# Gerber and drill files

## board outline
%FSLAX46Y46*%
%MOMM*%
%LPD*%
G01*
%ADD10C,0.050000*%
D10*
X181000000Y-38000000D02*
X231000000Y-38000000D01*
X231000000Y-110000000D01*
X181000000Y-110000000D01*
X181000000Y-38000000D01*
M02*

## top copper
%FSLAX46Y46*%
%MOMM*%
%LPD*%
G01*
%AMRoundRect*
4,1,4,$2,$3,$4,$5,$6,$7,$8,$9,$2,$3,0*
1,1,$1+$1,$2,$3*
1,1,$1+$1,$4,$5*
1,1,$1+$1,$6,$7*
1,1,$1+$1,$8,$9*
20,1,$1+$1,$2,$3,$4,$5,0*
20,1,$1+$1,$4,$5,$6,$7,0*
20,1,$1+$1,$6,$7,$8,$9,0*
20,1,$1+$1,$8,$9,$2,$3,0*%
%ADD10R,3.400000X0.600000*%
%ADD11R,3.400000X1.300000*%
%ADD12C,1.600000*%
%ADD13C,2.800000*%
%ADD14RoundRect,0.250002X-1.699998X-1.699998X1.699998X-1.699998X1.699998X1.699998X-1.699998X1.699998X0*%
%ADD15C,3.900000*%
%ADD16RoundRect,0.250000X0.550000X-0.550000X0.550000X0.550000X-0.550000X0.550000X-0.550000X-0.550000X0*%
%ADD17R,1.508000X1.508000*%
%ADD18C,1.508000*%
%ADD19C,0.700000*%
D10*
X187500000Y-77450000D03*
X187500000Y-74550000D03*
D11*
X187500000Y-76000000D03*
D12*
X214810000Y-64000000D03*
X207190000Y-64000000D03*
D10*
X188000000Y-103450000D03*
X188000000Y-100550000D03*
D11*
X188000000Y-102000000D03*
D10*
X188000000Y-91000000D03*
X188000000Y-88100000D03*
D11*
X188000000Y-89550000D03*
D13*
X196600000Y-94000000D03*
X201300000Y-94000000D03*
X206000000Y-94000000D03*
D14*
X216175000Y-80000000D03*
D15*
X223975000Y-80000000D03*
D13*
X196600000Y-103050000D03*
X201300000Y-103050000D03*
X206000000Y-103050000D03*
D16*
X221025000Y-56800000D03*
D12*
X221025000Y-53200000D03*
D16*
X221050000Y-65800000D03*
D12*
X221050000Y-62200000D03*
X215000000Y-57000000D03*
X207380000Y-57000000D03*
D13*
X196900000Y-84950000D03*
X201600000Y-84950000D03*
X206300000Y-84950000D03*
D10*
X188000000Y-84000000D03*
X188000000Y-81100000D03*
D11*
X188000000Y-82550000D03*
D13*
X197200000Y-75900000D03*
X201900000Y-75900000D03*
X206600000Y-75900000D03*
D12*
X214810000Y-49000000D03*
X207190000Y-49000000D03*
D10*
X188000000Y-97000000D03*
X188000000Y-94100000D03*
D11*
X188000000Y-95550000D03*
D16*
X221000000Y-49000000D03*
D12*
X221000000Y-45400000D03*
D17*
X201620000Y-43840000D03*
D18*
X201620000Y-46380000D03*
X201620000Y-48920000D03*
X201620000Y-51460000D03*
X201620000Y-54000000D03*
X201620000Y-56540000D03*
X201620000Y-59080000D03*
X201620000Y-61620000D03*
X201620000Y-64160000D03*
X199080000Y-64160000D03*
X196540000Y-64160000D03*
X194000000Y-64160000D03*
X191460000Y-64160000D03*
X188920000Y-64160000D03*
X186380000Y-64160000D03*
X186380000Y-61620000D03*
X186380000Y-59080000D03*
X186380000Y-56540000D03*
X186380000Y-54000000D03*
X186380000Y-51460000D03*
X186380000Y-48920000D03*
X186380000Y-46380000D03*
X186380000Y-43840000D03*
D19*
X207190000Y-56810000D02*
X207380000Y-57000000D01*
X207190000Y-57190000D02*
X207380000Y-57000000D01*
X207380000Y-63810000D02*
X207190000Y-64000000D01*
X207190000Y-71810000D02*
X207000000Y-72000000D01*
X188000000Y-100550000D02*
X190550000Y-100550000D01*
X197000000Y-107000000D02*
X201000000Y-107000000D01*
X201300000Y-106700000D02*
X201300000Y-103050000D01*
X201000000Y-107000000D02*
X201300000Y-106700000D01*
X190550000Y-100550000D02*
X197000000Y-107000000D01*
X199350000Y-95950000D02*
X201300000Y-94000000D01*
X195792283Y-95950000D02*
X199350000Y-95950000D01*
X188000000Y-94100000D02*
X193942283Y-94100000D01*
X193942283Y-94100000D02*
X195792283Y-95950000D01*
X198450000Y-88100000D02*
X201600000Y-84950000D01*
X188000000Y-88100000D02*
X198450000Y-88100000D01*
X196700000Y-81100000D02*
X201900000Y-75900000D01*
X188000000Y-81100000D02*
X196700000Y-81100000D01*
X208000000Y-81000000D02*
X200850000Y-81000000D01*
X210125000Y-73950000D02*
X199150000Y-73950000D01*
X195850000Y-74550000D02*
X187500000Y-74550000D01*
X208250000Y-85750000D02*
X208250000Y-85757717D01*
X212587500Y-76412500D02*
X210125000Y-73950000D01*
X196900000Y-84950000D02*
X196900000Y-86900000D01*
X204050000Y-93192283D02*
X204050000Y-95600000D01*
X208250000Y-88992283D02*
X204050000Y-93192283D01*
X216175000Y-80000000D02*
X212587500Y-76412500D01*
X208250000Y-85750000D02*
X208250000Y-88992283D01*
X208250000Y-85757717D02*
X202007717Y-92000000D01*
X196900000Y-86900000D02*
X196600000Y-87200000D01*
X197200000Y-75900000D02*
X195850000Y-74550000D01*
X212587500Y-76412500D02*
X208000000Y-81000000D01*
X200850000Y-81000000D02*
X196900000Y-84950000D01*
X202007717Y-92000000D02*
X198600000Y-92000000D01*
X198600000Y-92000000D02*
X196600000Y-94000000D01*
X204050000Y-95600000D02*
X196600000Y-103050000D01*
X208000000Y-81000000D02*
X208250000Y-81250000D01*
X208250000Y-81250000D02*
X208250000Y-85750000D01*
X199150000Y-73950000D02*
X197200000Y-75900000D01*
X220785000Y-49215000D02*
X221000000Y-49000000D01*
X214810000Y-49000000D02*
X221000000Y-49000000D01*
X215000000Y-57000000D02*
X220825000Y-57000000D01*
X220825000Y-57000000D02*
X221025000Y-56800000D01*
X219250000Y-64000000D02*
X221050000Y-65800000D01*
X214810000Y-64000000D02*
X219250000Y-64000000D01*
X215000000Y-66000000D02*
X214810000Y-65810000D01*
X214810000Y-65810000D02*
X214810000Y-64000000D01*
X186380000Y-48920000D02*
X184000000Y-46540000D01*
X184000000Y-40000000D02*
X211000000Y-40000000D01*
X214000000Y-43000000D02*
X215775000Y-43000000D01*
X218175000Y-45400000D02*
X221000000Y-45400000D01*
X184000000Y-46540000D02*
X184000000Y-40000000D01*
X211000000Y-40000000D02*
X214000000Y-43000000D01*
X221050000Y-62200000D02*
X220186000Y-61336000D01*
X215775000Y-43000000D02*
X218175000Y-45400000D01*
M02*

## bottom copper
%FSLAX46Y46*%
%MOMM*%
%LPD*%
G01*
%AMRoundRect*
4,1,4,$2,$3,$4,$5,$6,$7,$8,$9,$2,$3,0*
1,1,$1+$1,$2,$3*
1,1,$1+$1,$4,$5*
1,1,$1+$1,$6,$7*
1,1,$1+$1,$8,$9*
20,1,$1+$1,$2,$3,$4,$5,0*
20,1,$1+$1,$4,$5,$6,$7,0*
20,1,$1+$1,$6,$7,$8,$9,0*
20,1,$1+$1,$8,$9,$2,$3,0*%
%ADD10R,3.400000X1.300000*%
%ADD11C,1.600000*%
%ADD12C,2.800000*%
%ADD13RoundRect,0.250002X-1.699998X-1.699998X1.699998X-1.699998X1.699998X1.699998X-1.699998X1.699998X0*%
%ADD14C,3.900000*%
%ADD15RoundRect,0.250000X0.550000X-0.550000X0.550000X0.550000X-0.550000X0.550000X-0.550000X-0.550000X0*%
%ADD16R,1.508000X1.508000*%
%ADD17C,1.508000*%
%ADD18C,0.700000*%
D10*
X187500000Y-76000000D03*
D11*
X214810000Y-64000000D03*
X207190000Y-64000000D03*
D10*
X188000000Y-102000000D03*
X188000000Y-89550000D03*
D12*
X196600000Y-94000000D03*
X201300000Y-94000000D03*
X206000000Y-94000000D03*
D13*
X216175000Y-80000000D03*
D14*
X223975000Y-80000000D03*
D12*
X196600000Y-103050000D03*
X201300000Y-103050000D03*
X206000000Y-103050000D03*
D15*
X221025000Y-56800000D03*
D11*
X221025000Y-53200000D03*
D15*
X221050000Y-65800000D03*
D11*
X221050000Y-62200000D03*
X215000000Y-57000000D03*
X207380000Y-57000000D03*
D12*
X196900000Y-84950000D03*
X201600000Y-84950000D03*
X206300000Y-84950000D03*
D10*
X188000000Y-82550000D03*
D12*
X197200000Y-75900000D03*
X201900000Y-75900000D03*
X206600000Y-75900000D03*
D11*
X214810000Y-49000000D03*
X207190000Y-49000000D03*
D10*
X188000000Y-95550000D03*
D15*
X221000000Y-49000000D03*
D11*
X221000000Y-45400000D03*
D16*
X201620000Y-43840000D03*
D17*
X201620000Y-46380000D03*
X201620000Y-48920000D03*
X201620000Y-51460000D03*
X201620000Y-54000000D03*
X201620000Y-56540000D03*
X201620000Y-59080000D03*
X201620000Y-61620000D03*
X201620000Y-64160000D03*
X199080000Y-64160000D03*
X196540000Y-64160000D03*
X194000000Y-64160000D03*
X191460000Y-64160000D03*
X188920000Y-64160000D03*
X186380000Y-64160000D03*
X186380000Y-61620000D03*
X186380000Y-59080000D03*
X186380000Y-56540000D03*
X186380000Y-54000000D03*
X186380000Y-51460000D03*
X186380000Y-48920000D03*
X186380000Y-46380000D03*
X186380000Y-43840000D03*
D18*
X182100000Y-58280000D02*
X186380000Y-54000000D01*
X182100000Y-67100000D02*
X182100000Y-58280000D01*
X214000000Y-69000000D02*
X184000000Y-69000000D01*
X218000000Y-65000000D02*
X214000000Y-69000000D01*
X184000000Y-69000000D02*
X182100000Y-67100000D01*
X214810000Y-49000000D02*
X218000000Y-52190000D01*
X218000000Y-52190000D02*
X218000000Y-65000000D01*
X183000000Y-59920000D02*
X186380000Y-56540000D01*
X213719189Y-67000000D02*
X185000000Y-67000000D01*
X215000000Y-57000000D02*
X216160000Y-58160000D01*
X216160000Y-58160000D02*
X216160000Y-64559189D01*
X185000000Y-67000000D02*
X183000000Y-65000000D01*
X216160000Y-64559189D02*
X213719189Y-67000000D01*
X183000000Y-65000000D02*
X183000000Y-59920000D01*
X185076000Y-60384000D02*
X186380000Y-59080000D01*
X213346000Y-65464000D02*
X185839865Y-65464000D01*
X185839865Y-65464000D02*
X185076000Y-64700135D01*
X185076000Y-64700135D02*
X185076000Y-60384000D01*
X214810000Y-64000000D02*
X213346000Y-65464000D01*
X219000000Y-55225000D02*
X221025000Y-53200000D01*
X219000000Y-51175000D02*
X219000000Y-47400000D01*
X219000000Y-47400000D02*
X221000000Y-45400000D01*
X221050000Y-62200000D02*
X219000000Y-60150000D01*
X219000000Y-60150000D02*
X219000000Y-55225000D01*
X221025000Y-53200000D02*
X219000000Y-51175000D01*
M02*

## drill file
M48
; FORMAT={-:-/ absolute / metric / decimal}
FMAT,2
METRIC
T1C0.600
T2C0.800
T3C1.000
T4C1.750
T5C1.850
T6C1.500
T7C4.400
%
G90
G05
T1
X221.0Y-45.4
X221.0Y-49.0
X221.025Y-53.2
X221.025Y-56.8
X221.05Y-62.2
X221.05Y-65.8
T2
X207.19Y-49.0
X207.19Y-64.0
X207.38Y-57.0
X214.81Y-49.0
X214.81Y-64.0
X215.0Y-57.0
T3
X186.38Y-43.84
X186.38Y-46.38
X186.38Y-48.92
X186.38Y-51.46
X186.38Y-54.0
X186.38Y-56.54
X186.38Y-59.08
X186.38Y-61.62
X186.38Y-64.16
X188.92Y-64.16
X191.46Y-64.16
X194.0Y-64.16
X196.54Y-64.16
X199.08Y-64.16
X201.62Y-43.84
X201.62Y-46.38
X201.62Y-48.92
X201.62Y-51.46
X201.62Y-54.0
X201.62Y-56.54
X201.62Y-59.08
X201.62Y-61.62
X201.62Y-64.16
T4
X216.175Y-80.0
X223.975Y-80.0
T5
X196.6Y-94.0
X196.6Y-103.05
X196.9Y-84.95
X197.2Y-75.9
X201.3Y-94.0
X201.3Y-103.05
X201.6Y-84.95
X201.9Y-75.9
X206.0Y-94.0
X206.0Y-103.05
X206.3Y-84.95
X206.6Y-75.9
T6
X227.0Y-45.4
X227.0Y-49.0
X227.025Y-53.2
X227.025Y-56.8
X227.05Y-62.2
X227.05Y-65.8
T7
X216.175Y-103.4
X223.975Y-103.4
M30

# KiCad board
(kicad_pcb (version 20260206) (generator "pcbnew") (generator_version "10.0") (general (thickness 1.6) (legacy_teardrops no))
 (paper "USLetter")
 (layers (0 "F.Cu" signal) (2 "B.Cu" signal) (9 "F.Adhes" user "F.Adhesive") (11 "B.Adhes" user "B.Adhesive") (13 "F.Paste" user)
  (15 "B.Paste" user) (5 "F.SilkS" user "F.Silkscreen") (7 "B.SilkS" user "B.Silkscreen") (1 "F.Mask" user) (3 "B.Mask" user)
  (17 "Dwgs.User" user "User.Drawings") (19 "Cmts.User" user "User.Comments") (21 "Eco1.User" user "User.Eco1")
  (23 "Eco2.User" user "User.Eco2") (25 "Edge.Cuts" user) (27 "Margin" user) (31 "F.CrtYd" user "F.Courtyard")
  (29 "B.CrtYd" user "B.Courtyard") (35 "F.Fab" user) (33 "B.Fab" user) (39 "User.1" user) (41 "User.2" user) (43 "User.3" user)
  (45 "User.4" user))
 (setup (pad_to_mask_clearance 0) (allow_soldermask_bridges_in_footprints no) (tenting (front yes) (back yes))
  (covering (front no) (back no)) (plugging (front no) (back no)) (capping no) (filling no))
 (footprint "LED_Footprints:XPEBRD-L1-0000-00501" (layer "F.Cu") (at 187.5 76 90)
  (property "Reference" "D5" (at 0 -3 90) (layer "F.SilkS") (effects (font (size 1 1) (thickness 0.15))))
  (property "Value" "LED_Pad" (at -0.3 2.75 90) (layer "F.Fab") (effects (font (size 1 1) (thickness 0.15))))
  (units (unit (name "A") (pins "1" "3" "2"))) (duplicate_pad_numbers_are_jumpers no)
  (pad "" smd rect (at 0 0 90) (size 1 3) (layers "F.Paste"))
  (pad "1" smd rect (at -1.45 0 90) (size 0.6 3.4) (layers "F.Cu" "F.Mask" "F.Paste") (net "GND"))
  (pad "2" smd rect (at 1.45 0 90) (size 0.6 3.4) (layers "F.Cu" "F.Mask" "F.Paste") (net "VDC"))
  (pad "3" smd rect (at 0 0 90) (size 1.3 3.4) (layers "F.Cu" "F.Mask") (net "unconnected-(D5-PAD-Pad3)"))
  (pad "3" smd rect (at 0 0 90) (size 1.3 3.4) (layers "B.Cu" "B.Mask") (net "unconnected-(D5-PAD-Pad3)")))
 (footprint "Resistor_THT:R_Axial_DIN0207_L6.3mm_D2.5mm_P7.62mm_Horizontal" (layer "F.Cu") (at 214.81 64 180)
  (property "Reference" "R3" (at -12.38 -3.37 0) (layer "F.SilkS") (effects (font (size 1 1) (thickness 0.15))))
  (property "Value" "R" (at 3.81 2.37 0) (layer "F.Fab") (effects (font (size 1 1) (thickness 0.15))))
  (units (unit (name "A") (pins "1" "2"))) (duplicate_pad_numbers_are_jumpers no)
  (pad "1" thru_hole circle (at 0 0 180) (size 1.6 1.6) (drill 0.8) (layers "*.Cu" "*.Mask") (remove_unused_layers no)
   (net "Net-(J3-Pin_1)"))
  (pad "2" thru_hole circle (at 7.62 0 180) (size 1.6 1.6) (drill 0.8) (layers "*.Cu" "*.Mask") (remove_unused_layers no) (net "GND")))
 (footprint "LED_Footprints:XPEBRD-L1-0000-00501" (layer "F.Cu") (at 188 102 90)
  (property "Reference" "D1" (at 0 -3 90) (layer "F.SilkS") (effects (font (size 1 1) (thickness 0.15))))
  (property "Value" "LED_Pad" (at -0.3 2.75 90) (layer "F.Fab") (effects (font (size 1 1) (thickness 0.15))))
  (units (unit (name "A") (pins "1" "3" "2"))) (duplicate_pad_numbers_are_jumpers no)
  (pad "" smd rect (at 0 0 90) (size 1 3) (layers "F.Paste"))
  (pad "1" smd rect (at -1.45 0 90) (size 0.6 3.4) (layers "F.Cu" "F.Mask" "F.Paste") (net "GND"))
  (pad "2" smd rect (at 1.45 0 90) (size 0.6 3.4) (layers "F.Cu" "F.Mask" "F.Paste") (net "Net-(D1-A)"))
  (pad "3" smd rect (at 0 0 90) (size 1.3 3.4) (layers "F.Cu" "F.Mask") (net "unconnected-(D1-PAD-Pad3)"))
  (pad "3" smd rect (at 0 0 90) (size 1.3 3.4) (layers "B.Cu" "B.Mask") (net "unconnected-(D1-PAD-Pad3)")))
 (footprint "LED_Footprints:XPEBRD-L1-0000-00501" (layer "F.Cu") (at 188 89.55 90)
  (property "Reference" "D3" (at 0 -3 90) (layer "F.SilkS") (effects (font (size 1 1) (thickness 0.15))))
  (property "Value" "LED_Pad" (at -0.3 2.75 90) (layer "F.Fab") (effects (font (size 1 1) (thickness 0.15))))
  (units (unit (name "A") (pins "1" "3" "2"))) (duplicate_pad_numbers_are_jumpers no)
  (pad "" smd rect (at 0 0 90) (size 1 3) (layers "F.Paste"))
  (pad "1" smd rect (at -1.45 0 90) (size 0.6 3.4) (layers "F.Cu" "F.Mask" "F.Paste") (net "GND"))
  (pad "2" smd rect (at 1.45 0 90) (size 0.6 3.4) (layers "F.Cu" "F.Mask" "F.Paste") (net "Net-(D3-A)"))
  (pad "3" smd rect (at 0 0 90) (size 1.3 3.4) (layers "F.Cu" "F.Mask") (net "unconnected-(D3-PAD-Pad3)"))
  (pad "3" smd rect (at 0 0 90) (size 1.3 3.4) (layers "B.Cu" "B.Mask") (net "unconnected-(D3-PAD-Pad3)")))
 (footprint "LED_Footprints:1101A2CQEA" (layer "F.Cu") (at 201.3 94)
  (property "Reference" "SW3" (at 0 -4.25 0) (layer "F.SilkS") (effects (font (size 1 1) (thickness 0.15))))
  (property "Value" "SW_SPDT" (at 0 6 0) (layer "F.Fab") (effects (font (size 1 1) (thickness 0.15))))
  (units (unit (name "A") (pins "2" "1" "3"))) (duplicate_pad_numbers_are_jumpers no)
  (pad "1" thru_hole circle (at -4.7 0) (size 2.8 2.8) (drill 1.85) (layers "*.Cu" "*.Mask") (remove_unused_layers no) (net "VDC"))
  (pad "2" thru_hole circle (at 0 0) (size 2.8 2.8) (drill 1.85) (layers "*.Cu" "*.Mask") (remove_unused_layers no) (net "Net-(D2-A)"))
  (pad "3" thru_hole circle (at 4.7 0) (size 2.8 2.8) (drill 1.85) (layers "*.Cu" "*.Mask") (remove_unused_layers no)
   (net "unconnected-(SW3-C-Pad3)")))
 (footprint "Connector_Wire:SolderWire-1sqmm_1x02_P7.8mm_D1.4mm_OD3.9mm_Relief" (layer "F.Cu") (at 216.175 80)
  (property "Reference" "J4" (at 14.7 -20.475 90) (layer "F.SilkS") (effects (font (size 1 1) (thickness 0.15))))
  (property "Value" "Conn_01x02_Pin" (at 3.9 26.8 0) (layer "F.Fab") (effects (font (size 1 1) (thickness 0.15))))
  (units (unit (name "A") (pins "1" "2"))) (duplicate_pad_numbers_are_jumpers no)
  (pad "" np_thru_hole circle (at 0 23.4) (size 4.4 4.4) (drill 4.4) (layers "*.Cu" "*.Mask"))
  (pad "" np_thru_hole circle (at 7.8 23.4) (size 4.4 4.4) (drill 4.4) (layers "*.Cu" "*.Mask"))
  (pad "1" thru_hole roundrect (at 0 0) (size 3.9 3.9) (drill 1.75) (layers "*.Cu" "*.Mask") (remove_unused_layers no)
   (roundrect_rratio 0.064103) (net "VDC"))
  (pad "2" thru_hole circle (at 7.8 0) (size 3.9 3.9) (drill 1.75) (layers "*.Cu" "*.Mask") (remove_unused_layers no) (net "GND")))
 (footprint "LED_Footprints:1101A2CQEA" (layer "F.Cu") (at 201.3 103.05)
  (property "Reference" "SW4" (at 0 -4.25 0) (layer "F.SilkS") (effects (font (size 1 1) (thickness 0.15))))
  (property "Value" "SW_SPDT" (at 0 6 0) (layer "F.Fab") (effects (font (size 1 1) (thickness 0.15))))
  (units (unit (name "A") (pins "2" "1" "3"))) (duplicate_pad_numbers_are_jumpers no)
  (pad "1" thru_hole circle (at -4.7 0) (size 2.8 2.8) (drill 1.85) (layers "*.Cu" "*.Mask") (remove_unused_layers no) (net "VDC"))
  (pad "2" thru_hole circle (at 0 0) (size 2.8 2.8) (drill 1.85) (layers "*.Cu" "*.Mask") (remove_unused_layers no) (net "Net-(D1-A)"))
  (pad "3" thru_hole circle (at 4.7 0) (size 2.8 2.8) (drill 1.85) (layers "*.Cu" "*.Mask") (remove_unused_layers no)
   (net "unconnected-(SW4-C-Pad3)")))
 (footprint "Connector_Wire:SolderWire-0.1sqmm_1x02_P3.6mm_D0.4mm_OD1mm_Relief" (layer "F.Cu") (at 221.025 56.8 90)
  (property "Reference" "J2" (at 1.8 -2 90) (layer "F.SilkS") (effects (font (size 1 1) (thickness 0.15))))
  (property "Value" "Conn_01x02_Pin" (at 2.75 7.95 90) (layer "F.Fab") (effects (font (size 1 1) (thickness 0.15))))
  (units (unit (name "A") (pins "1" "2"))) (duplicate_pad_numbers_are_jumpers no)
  (pad "" np_thru_hole circle (at 0 6 90) (size 1.5 1.5) (drill 1.5) (layers "*.Cu" "*.Mask"))
  (pad "" np_thru_hole circle (at 3.6 6 90) (size 1.5 1.5) (drill 1.5) (layers "*.Cu" "*.Mask"))
  (pad "1" thru_hole roundrect (at 0 0 90) (size 1.6 1.6) (drill 0.6) (layers "*.Cu" "*.Mask") (remove_unused_layers no)
   (roundrect_rratio 0.15625) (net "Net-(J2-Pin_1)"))
  (pad "2" thru_hole circle (at 3.6 0 90) (size 1.6 1.6) (drill 0.6) (layers "*.Cu" "*.Mask") (remove_unused_layers no)
   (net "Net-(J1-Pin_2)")))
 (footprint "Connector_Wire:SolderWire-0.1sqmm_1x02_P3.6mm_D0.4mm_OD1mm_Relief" (layer "F.Cu") (at 221.05 65.8 90)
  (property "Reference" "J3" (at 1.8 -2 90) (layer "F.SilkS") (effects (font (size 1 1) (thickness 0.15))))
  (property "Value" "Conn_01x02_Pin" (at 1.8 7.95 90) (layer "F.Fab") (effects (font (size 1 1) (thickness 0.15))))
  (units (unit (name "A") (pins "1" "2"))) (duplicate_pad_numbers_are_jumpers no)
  (pad "" np_thru_hole circle (at 0 6 90) (size 1.5 1.5) (drill 1.5) (layers "*.Cu" "*.Mask"))
  (pad "" np_thru_hole circle (at 3.6 6 90) (size 1.5 1.5) (drill 1.5) (layers "*.Cu" "*.Mask"))
  (pad "1" thru_hole roundrect (at 0 0 90) (size 1.6 1.6) (drill 0.6) (layers "*.Cu" "*.Mask") (remove_unused_layers no)
   (roundrect_rratio 0.15625) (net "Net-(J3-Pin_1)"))
  (pad "2" thru_hole circle (at 3.6 0 90) (size 1.6 1.6) (drill 0.6) (layers "*.Cu" "*.Mask") (remove_unused_layers no)
   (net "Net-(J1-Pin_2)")))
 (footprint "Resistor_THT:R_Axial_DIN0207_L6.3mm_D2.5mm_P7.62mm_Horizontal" (layer "F.Cu") (at 215 57 180)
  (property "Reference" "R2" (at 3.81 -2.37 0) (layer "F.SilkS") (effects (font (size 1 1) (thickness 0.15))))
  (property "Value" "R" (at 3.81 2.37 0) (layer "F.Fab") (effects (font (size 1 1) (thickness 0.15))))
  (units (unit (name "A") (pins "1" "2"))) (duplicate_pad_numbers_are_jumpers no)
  (pad "1" thru_hole circle (at 0 0 180) (size 1.6 1.6) (drill 0.8) (layers "*.Cu" "*.Mask") (remove_unused_layers no)
   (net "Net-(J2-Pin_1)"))
  (pad "2" thru_hole circle (at 7.62 0 180) (size 1.6 1.6) (drill 0.8) (layers "*.Cu" "*.Mask") (remove_unused_layers no) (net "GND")))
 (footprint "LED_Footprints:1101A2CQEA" (layer "F.Cu") (at 201.6 84.95)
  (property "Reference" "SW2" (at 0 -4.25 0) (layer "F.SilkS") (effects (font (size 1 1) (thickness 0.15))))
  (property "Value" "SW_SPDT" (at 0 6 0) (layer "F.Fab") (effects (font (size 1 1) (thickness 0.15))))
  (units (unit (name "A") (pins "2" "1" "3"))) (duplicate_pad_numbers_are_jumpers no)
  (pad "1" thru_hole circle (at -4.7 0) (size 2.8 2.8) (drill 1.85) (layers "*.Cu" "*.Mask") (remove_unused_layers no) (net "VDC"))
  (pad "2" thru_hole circle (at 0 0) (size 2.8 2.8) (drill 1.85) (layers "*.Cu" "*.Mask") (remove_unused_layers no) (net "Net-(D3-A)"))
  (pad "3" thru_hole circle (at 4.7 0) (size 2.8 2.8) (drill 1.85) (layers "*.Cu" "*.Mask") (remove_unused_layers no)
   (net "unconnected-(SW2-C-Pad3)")))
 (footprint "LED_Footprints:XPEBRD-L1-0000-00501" (layer "F.Cu") (at 188 82.55 90)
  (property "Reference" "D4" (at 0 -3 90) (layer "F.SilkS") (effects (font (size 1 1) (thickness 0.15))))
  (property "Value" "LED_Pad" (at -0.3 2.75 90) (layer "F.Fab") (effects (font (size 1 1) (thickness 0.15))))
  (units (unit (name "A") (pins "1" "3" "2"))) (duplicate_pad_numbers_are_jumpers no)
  (pad "" smd rect (at 0 0 90) (size 1 3) (layers "F.Paste"))
  (pad "1" smd rect (at -1.45 0 90) (size 0.6 3.4) (layers "F.Cu" "F.Mask" "F.Paste") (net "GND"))
  (pad "2" smd rect (at 1.45 0 90) (size 0.6 3.4) (layers "F.Cu" "F.Mask" "F.Paste") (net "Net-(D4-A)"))
  (pad "3" smd rect (at 0 0 90) (size 1.3 3.4) (layers "F.Cu" "F.Mask") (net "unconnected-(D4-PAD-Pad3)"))
  (pad "3" smd rect (at 0 0 90) (size 1.3 3.4) (layers "B.Cu" "B.Mask") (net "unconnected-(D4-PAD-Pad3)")))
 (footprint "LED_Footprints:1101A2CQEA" (layer "F.Cu") (at 201.9 75.9)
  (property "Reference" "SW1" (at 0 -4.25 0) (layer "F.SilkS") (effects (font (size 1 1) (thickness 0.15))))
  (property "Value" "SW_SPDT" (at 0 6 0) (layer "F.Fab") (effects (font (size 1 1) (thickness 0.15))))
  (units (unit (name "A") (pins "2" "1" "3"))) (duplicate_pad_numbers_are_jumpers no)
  (pad "1" thru_hole circle (at -4.7 0) (size 2.8 2.8) (drill 1.85) (layers "*.Cu" "*.Mask") (remove_unused_layers no) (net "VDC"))
  (pad "2" thru_hole circle (at 0 0) (size 2.8 2.8) (drill 1.85) (layers "*.Cu" "*.Mask") (remove_unused_layers no) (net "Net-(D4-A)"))
  (pad "3" thru_hole circle (at 4.7 0) (size 2.8 2.8) (drill 1.85) (layers "*.Cu" "*.Mask") (remove_unused_layers no)
   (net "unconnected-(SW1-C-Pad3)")))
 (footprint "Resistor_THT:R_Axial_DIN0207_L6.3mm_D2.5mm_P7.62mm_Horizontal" (layer "F.Cu") (at 214.81 49 180)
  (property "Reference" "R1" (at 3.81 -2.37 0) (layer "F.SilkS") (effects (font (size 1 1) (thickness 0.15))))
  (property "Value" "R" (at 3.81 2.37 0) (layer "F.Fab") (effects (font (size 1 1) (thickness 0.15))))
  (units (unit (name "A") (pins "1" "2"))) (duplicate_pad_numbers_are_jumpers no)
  (pad "1" thru_hole circle (at 0 0 180) (size 1.6 1.6) (drill 0.8) (layers "*.Cu" "*.Mask") (remove_unused_layers no)
   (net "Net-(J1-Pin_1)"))
  (pad "2" thru_hole circle (at 7.62 0 180) (size 1.6 1.6) (drill 0.8) (layers "*.Cu" "*.Mask") (remove_unused_layers no) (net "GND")))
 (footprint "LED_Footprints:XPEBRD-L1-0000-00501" (layer "F.Cu") (at 188 95.55 90)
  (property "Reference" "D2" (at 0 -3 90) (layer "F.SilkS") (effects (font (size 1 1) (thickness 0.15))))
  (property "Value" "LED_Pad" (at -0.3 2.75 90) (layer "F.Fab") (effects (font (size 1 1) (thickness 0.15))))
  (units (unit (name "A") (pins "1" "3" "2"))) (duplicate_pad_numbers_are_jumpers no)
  (pad "" smd rect (at 0 0 90) (size 1 3) (layers "F.Paste"))
  (pad "1" smd rect (at -1.45 0 90) (size 0.6 3.4) (layers "F.Cu" "F.Mask" "F.Paste") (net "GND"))
  (pad "2" smd rect (at 1.45 0 90) (size 0.6 3.4) (layers "F.Cu" "F.Mask" "F.Paste") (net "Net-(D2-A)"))
  (pad "3" smd rect (at 0 0 90) (size 1.3 3.4) (layers "F.Cu" "F.Mask") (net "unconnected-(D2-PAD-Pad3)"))
  (pad "3" smd rect (at 0 0 90) (size 1.3 3.4) (layers "B.Cu" "B.Mask") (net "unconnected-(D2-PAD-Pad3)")))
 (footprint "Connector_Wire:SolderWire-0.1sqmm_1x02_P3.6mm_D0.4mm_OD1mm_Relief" (layer "F.Cu") (at 221 49 90)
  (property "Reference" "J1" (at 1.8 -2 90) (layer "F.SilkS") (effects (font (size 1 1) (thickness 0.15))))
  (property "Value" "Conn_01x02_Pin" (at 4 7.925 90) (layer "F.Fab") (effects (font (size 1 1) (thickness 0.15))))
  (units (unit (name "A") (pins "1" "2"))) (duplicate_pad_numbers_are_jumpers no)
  (pad "" np_thru_hole circle (at 0 6 90) (size 1.5 1.5) (drill 1.5) (layers "*.Cu" "*.Mask"))
  (pad "" np_thru_hole circle (at 3.6 6 90) (size 1.5 1.5) (drill 1.5) (layers "*.Cu" "*.Mask"))
  (pad "1" thru_hole roundrect (at 0 0 90) (size 1.6 1.6) (drill 0.6) (layers "*.Cu" "*.Mask") (remove_unused_layers no)
   (roundrect_rratio 0.15625) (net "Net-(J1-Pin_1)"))
  (pad "2" thru_hole circle (at 3.6 0 90) (size 1.6 1.6) (drill 0.6) (layers "*.Cu" "*.Mask") (remove_unused_layers no)
   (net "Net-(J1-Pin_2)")))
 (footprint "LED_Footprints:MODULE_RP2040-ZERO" (layer "F.Cu") (at 194 54)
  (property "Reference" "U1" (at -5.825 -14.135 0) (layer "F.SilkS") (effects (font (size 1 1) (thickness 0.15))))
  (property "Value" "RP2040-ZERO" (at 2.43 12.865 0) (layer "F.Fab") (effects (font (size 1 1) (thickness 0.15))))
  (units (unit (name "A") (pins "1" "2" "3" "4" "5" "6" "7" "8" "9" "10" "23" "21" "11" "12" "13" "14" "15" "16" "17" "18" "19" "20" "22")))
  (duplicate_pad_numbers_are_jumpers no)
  (pad "1" thru_hole rect (at 7.62 -10.16) (size 1.508 1.508) (drill 1) (layers "*.Cu" "*.Mask") (remove_unused_layers no)
   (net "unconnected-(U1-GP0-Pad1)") (solder_mask_margin 0.102))
  (pad "2" thru_hole circle (at 7.62 -7.62) (size 1.508 1.508) (drill 1) (layers "*.Cu" "*.Mask") (remove_unused_layers no)
   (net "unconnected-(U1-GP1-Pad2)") (solder_mask_margin 0.102))
  (pad "3" thru_hole circle (at 7.62 -5.08) (size 1.508 1.508) (drill 1) (layers "*.Cu" "*.Mask") (remove_unused_layers no)
   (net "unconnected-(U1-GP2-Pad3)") (solder_mask_margin 0.102))
  (pad "4" thru_hole circle (at 7.62 -2.54) (size 1.508 1.508) (drill 1) (layers "*.Cu" "*.Mask") (remove_unused_layers no)
   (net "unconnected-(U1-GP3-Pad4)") (solder_mask_margin 0.102))
  (pad "5" thru_hole circle (at 7.62 0) (size 1.508 1.508) (drill 1) (layers "*.Cu" "*.Mask") (remove_unused_layers no)
   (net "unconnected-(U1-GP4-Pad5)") (solder_mask_margin 0.102))
  (pad "6" thru_hole circle (at 7.62 2.54) (size 1.508 1.508) (drill 1) (layers "*.Cu" "*.Mask") (remove_unused_layers no)
   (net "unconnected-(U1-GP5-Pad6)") (solder_mask_margin 0.102))
  (pad "7" thru_hole circle (at 7.62 5.08) (size 1.508 1.508) (drill 1) (layers "*.Cu" "*.Mask") (remove_unused_layers no)
   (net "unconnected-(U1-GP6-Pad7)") (solder_mask_margin 0.102))
  (pad "8" thru_hole circle (at 7.62 7.62) (size 1.508 1.508) (drill 1) (layers "*.Cu" "*.Mask") (remove_unused_layers no)
   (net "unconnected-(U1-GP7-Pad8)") (solder_mask_margin 0.102))
  (pad "9" thru_hole circle (at 7.62 10.16) (size 1.508 1.508) (drill 1) (layers "*.Cu" "*.Mask") (remove_unused_layers no)
   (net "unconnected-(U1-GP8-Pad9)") (solder_mask_margin 0.102))
  (pad "10" thru_hole circle (at 5.08 10.16) (size 1.508 1.508) (drill 1) (layers "*.Cu" "*.Mask") (remove_unused_layers no)
   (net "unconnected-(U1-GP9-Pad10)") (solder_mask_margin 0.102))
  (pad "11" thru_hole circle (at 2.54 10.16) (size 1.508 1.508) (drill 1) (layers "*.Cu" "*.Mask") (remove_unused_layers no)
   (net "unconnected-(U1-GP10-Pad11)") (solder_mask_margin 0.102))
  (pad "12" thru_hole circle (at 0 10.16) (size 1.508 1.508) (drill 1) (layers "*.Cu" "*.Mask") (remove_unused_layers no)
   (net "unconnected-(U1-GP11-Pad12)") (solder_mask_margin 0.102))
  (pad "13" thru_hole circle (at -2.54 10.16) (size 1.508 1.508) (drill 1) (layers "*.Cu" "*.Mask") (remove_unused_layers no)
   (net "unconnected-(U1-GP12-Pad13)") (solder_mask_margin 0.102))
  (pad "14" thru_hole circle (at -5.08 10.16) (size 1.508 1.508) (drill 1) (layers "*.Cu" "*.Mask") (remove_unused_layers no)
   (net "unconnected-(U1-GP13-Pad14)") (solder_mask_margin 0.102))
  (pad "15" thru_hole circle (at -7.62 10.16) (size 1.508 1.508) (drill 1) (layers "*.Cu" "*.Mask") (remove_unused_layers no)
   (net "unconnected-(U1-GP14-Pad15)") (solder_mask_margin 0.102))
  (pad "16" thru_hole circle (at -7.62 7.62) (size 1.508 1.508) (drill 1) (layers "*.Cu" "*.Mask") (remove_unused_layers no)
   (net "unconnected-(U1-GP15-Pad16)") (solder_mask_margin 0.102))
  (pad "17" thru_hole circle (at -7.62 5.08) (size 1.508 1.508) (drill 1) (layers "*.Cu" "*.Mask") (remove_unused_layers no)
   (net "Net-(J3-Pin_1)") (solder_mask_margin 0.102))
  (pad "18" thru_hole circle (at -7.62 2.54) (size 1.508 1.508) (drill 1) (layers "*.Cu" "*.Mask") (remove_unused_layers no)
   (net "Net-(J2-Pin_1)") (solder_mask_margin 0.102))
  (pad "19" thru_hole circle (at -7.62 0) (size 1.508 1.508) (drill 1) (layers "*.Cu" "*.Mask") (remove_unused_layers no)
   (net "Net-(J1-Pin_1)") (solder_mask_margin 0.102))
  (pad "20" thru_hole circle (at -7.62 -2.54) (size 1.508 1.508) (drill 1) (layers "*.Cu" "*.Mask") (remove_unused_layers no)
   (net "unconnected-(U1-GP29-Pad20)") (solder_mask_margin 0.102))
  (pad "21" thru_hole circle (at -7.62 -5.08) (size 1.508 1.508) (drill 1) (layers "*.Cu" "*.Mask") (remove_unused_layers no)
   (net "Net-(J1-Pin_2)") (solder_mask_margin 0.102))
  (pad "22" thru_hole circle (at -7.62 -7.62) (size 1.508 1.508) (drill 1) (layers "*.Cu" "*.Mask") (remove_unused_layers no)
   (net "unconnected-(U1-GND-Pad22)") (solder_mask_margin 0.102))
  (pad "23" thru_hole circle (at -7.62 -10.16) (size 1.508 1.508) (drill 1) (layers "*.Cu" "*.Mask") (remove_unused_layers no)
   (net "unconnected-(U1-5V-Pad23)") (solder_mask_margin 0.102)))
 (gr_rect (start 181 38) (end 231 110) (stroke (width 0.05) (type default)) (fill no) (layer "Edge.Cuts"))
 (segment (start 207.19 56.81) (end 207.38 57) (width 0.7) (layer "F.Cu") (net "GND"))
 (segment (start 207.19 57.19) (end 207.38 57) (width 0.7) (layer "F.Cu") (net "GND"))
 (segment (start 207.38 63.81) (end 207.19 64) (width 0.7) (layer "F.Cu") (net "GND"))
 (segment (start 207.19 71.81) (end 207 72) (width 0.7) (layer "F.Cu") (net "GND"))
 (segment (start 188 100.55) (end 190.55 100.55) (width 0.7) (layer "F.Cu") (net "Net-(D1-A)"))
 (segment (start 197 107) (end 201 107) (width 0.7) (layer "F.Cu") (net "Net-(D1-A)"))
 (segment (start 201.3 106.7) (end 201.3 103.05) (width 0.7) (layer "F.Cu") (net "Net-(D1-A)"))
 (segment (start 201 107) (end 201.3 106.7) (width 0.7) (layer "F.Cu") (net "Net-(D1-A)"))
 (segment (start 190.55 100.55) (end 197 107) (width 0.7) (layer "F.Cu") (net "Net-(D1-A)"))
 (segment (start 199.35 95.95) (end 201.3 94) (width 0.7) (layer "F.Cu") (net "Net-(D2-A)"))
 (segment (start 195.792283 95.95) (end 199.35 95.95) (width 0.7) (layer "F.Cu") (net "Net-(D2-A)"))
 (segment (start 188 94.1) (end 193.942283 94.1) (width 0.7) (layer "F.Cu") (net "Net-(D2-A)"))
 (segment (start 193.942283 94.1) (end 195.792283 95.95) (width 0.7) (layer "F.Cu") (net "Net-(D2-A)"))
 (segment (start 198.45 88.1) (end 201.6 84.95) (width 0.7) (layer "F.Cu") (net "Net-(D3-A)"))
 (segment (start 188 88.1) (end 198.45 88.1) (width 0.7) (layer "F.Cu") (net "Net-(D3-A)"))
 (segment (start 196.7 81.1) (end 201.9 75.9) (width 0.7) (layer "F.Cu") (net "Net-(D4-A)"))
 (segment (start 188 81.1) (end 196.7 81.1) (width 0.7) (layer "F.Cu") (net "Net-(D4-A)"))
 (segment (start 208 81) (end 200.85 81) (width 0.7) (layer "F.Cu") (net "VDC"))
 (segment (start 210.125 73.95) (end 199.15 73.95) (width 0.7) (layer "F.Cu") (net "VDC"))
 (segment (start 195.85 74.55) (end 187.5 74.55) (width 0.7) (layer "F.Cu") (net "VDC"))
 (segment (start 208.25 85.75) (end 208.25 85.757717) (width 0.7) (layer "F.Cu") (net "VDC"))
 (segment (start 212.5875 76.4125) (end 210.125 73.95) (width 0.7) (layer "F.Cu") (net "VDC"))
 (segment (start 196.9 84.95) (end 196.9 86.9) (width 0.7) (layer "F.Cu") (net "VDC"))
 (segment (start 204.05 93.192283) (end 204.05 95.6) (width 0.7) (layer "F.Cu") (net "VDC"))
 (segment (start 208.25 88.992283) (end 204.05 93.192283) (width 0.7) (layer "F.Cu") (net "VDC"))
 (segment (start 216.175 80) (end 212.5875 76.4125) (width 0.7) (layer "F.Cu") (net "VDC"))
 (segment (start 208.25 85.75) (end 208.25 88.992283) (width 0.7) (layer "F.Cu") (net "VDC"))
 (segment (start 208.25 85.757717) (end 202.007717 92) (width 0.7) (layer "F.Cu") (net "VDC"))
 (segment (start 196.9 86.9) (end 196.6 87.2) (width 0.7) (layer "F.Cu") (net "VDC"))
 (segment (start 197.2 75.9) (end 195.85 74.55) (width 0.7) (layer "F.Cu") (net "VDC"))
 (segment (start 212.5875 76.4125) (end 208 81) (width 0.7) (layer "F.Cu") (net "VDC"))
 (segment (start 200.85 81) (end 196.9 84.95) (width 0.7) (layer "F.Cu") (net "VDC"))
 (segment (start 202.007717 92) (end 198.6 92) (width 0.7) (layer "F.Cu") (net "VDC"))
 (segment (start 198.6 92) (end 196.6 94) (width 0.7) (layer "F.Cu") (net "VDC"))
 (segment (start 204.05 95.6) (end 196.6 103.05) (width 0.7) (layer "F.Cu") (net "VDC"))
 (segment (start 208 81) (end 208.25 81.25) (width 0.7) (layer "F.Cu") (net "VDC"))
 (segment (start 208.25 81.25) (end 208.25 85.75) (width 0.7) (layer "F.Cu") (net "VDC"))
 (segment (start 199.15 73.95) (end 197.2 75.9) (width 0.7) (layer "F.Cu") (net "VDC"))
 (segment (start 220.785 49.215) (end 221 49) (width 0.7) (layer "F.Cu") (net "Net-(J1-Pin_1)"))
 (segment (start 214.81 49) (end 221 49) (width 0.7) (layer "F.Cu") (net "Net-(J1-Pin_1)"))
 (segment (start 182.1 58.28) (end 186.38 54) (width 0.7) (layer "B.Cu") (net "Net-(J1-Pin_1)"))
 (segment (start 182.1 67.1) (end 182.1 58.28) (width 0.7) (layer "B.Cu") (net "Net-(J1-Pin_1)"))
 (segment (start 214 69) (end 184 69) (width 0.7) (layer "B.Cu") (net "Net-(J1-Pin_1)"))
 (segment (start 218 65) (end 214 69) (width 0.7) (layer "B.Cu") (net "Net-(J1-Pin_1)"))
 (segment (start 184 69) (end 182.1 67.1) (width 0.7) (layer "B.Cu") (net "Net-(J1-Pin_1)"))
 (segment (start 214.81 49) (end 218 52.19) (width 0.7) (layer "B.Cu") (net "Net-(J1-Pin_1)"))
 (segment (start 218 52.19) (end 218 65) (width 0.7) (layer "B.Cu") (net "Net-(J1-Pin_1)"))
 (segment (start 215 57) (end 220.825 57) (width 0.7) (layer "F.Cu") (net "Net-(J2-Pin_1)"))
 (segment (start 220.825 57) (end 221.025 56.8) (width 0.7) (layer "F.Cu") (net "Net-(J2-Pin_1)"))
 (segment (start 183 59.92) (end 186.38 56.54) (width 0.7) (layer "B.Cu") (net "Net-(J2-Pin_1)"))
 (segment (start 213.719189 67) (end 185 67) (width 0.7) (layer "B.Cu") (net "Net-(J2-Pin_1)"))
 (segment (start 215 57) (end 216.16 58.16) (width 0.7) (layer "B.Cu") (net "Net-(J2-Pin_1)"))
 (segment (start 216.16 58.16) (end 216.16 64.559189) (width 0.7) (layer "B.Cu") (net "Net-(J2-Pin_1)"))
 (segment (start 185 67) (end 183 65) (width 0.7) (layer "B.Cu") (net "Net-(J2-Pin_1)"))
 (segment (start 216.16 64.559189) (end 213.719189 67) (width 0.7) (layer "B.Cu") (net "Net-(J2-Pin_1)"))
 (segment (start 183 65) (end 183 59.92) (width 0.7) (layer "B.Cu") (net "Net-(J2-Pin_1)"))
 (segment (start 219.25 64) (end 221.05 65.8) (width 0.7) (layer "F.Cu") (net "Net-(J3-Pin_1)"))
 (segment (start 214.81 64) (end 219.25 64) (width 0.7) (layer "F.Cu") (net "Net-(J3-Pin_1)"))
 (segment (start 215 66) (end 214.81 65.81) (width 0.7) (layer "F.Cu") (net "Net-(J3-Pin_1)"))
 (segment (start 214.81 65.81) (end 214.81 64) (width 0.7) (layer "F.Cu") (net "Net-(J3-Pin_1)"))
 (segment (start 185.076 60.384) (end 186.38 59.08) (width 0.7) (layer "B.Cu") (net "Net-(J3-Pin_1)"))
 (segment (start 213.346 65.464) (end 185.839865 65.464) (width 0.7) (layer "B.Cu") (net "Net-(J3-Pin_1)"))
 (segment (start 185.839865 65.464) (end 185.076 64.700135) (width 0.7) (layer "B.Cu") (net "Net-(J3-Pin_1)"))
 (segment (start 185.076 64.700135) (end 185.076 60.384) (width 0.7) (layer "B.Cu") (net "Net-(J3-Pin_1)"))
 (segment (start 214.81 64) (end 213.346 65.464) (width 0.7) (layer "B.Cu") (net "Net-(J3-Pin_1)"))
 (segment (start 186.38 48.92) (end 184 46.54) (width 0.7) (layer "F.Cu") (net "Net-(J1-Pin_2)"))
 (segment (start 184 40) (end 211 40) (width 0.7) (layer "F.Cu") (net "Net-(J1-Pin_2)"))
 (segment (start 214 43) (end 215.775 43) (width 0.7) (layer "F.Cu") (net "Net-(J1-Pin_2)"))
 (segment (start 218.175 45.4) (end 221 45.4) (width 0.7) (layer "F.Cu") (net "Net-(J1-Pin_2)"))
 (segment (start 184 46.54) (end 184 40) (width 0.7) (layer "F.Cu") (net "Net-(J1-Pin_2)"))
 (segment (start 211 40) (end 214 43) (width 0.7) (layer "F.Cu") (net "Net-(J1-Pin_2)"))
 (segment (start 221.05 62.2) (end 220.186 61.336) (width 0.7) (layer "F.Cu") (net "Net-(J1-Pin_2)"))
 (segment (start 215.775 43) (end 218.175 45.4) (width 0.7) (layer "F.Cu") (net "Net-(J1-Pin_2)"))
 (segment (start 219 55.225) (end 221.025 53.2) (width 0.7) (layer "B.Cu") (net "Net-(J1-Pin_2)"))
 (segment (start 219 51.175) (end 219 47.4) (width 0.7) (layer "B.Cu") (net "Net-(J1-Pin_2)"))
 (segment (start 219 47.4) (end 221 45.4) (width 0.7) (layer "B.Cu") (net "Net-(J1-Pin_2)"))
 (segment (start 221.05 62.2) (end 219 60.15) (width 0.7) (layer "B.Cu") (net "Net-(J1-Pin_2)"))
 (segment (start 219 60.15) (end 219 55.225) (width 0.7) (layer "B.Cu") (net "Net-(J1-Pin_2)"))
 (segment (start 221.025 53.2) (end 219 51.175) (width 0.7) (layer "B.Cu") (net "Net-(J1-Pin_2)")))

